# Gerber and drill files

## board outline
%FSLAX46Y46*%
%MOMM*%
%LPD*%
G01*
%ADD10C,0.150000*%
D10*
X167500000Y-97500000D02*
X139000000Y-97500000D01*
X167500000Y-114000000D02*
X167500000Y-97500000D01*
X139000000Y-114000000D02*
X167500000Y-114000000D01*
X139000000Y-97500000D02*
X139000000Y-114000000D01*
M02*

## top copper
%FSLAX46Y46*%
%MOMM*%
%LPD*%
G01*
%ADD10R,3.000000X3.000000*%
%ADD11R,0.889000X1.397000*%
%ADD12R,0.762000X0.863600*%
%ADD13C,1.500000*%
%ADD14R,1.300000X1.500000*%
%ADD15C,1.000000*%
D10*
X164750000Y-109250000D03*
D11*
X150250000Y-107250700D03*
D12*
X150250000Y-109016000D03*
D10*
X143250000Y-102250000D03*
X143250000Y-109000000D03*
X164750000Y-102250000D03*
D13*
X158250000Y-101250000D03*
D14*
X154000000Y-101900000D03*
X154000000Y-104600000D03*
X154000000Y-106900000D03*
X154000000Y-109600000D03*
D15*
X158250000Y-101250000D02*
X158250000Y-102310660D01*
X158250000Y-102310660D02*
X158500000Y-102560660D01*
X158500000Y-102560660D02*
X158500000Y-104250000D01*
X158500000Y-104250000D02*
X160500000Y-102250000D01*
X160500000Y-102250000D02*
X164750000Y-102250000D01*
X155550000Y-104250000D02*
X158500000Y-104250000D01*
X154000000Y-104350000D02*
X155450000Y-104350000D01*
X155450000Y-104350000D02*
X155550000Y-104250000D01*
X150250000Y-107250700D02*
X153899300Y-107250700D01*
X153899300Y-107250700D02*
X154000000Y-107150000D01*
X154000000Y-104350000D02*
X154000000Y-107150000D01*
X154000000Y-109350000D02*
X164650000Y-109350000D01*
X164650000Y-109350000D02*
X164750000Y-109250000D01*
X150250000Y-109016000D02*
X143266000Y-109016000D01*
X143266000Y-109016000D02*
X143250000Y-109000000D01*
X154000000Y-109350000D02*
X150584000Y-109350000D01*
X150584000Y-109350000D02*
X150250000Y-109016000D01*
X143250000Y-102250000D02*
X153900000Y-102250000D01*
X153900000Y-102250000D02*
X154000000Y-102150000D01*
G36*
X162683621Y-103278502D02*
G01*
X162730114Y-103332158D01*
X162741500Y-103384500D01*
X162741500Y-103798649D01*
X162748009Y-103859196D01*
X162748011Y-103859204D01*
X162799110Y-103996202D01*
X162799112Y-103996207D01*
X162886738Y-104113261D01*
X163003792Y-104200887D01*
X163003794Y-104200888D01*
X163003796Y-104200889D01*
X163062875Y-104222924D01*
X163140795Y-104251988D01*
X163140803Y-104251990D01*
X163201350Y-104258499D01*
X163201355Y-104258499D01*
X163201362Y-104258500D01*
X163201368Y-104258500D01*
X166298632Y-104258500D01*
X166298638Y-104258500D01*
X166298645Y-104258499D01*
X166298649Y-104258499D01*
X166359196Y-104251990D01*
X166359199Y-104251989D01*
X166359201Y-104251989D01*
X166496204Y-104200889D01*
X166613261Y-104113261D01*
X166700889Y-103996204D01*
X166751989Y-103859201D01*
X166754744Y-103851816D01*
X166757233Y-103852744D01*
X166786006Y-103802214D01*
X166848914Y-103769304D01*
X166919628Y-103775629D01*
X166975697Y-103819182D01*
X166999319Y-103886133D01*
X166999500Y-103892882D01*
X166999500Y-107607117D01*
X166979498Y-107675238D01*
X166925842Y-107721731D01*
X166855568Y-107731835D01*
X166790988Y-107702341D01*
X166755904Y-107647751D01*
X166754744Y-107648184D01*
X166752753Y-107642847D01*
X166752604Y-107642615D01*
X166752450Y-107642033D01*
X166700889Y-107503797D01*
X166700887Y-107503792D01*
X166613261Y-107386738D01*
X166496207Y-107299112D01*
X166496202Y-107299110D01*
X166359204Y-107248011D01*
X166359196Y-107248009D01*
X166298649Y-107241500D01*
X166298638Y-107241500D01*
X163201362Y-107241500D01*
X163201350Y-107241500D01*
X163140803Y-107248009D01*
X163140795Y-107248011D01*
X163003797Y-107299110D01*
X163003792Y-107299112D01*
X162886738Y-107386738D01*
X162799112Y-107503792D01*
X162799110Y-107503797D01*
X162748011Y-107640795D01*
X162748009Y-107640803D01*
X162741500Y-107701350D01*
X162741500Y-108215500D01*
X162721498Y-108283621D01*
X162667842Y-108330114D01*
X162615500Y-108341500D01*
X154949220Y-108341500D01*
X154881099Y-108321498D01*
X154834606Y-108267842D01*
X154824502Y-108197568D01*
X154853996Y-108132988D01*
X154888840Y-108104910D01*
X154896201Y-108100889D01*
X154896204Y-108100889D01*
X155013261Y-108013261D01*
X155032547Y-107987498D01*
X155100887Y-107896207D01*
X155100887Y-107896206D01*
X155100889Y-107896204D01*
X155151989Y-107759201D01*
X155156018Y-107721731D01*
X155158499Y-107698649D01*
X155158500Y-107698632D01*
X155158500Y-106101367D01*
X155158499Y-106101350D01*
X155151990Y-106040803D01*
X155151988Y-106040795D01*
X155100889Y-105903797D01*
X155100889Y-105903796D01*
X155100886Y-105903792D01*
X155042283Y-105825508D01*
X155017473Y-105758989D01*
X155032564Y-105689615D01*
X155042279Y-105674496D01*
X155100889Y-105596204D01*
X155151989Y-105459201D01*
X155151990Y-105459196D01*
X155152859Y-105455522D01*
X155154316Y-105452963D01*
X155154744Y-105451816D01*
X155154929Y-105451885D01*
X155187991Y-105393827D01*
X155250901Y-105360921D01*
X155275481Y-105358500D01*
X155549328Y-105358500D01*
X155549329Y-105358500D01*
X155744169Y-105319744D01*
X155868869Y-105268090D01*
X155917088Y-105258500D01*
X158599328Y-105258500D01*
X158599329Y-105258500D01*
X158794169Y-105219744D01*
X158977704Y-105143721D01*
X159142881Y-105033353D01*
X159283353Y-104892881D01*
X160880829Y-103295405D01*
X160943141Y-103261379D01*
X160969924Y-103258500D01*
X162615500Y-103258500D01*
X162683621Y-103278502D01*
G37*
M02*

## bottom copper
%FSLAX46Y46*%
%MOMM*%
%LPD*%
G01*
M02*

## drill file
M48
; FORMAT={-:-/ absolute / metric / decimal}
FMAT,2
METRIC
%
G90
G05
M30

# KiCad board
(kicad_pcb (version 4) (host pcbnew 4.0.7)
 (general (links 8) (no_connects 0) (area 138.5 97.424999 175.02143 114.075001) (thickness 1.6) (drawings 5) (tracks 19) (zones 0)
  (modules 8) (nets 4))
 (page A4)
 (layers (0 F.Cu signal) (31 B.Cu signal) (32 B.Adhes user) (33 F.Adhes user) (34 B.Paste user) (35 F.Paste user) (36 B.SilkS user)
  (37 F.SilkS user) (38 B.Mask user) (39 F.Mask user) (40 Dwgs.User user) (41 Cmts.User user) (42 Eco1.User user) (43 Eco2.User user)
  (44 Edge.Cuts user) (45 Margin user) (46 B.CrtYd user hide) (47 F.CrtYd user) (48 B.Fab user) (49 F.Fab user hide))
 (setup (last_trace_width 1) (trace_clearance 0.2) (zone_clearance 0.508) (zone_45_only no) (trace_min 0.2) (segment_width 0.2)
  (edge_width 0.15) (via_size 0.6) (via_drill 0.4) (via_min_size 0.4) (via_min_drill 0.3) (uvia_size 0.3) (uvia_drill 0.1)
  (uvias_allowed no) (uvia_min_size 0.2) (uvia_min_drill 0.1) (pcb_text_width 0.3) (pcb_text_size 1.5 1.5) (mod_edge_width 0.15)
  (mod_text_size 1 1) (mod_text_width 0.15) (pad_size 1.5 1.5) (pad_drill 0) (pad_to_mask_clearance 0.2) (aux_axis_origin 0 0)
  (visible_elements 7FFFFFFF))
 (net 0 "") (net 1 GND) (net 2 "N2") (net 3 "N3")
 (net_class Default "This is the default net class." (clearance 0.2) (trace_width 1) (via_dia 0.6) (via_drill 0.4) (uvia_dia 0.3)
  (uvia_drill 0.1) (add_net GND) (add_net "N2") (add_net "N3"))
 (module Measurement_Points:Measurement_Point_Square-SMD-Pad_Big (layer F.Cu) (at 164.75 109.25)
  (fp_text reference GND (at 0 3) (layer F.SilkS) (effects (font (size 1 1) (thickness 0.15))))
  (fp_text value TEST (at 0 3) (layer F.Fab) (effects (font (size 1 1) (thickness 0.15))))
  (pad 1 smd rect (at 0 0) (size 3 3) (layers F.Cu F.Mask) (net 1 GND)))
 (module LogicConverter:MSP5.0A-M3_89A (layer F.Cu) (at 150.25 108 270)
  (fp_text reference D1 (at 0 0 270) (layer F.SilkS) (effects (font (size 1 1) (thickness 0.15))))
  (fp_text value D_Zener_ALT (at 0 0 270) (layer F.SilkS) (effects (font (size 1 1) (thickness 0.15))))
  (pad 1 smd rect (at -0.7493 0 270) (size 1.397 0.889) (layers F.Cu F.Paste F.Mask) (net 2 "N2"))
  (pad 2 smd rect (at 1.016 0 270) (size 0.8636 0.762) (layers F.Cu F.Paste F.Mask) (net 1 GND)))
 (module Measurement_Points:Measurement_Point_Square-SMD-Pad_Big (layer F.Cu) (at 143.25 102.25)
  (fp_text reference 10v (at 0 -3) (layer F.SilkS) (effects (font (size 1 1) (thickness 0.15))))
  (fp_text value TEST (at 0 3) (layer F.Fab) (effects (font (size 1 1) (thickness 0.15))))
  (pad 1 smd rect (at 0 0) (size 3 3) (layers F.Cu F.Mask) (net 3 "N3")))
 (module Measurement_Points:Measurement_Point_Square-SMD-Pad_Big (layer F.Cu) (at 143.25 109)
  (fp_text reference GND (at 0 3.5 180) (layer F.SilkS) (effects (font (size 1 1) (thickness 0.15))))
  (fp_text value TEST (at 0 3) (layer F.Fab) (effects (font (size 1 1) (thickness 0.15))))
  (pad 1 smd rect (at 0 0) (size 3 3) (layers F.Cu F.Mask) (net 1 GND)))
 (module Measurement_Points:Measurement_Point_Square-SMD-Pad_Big (layer F.Cu) (at 164.75 102.25)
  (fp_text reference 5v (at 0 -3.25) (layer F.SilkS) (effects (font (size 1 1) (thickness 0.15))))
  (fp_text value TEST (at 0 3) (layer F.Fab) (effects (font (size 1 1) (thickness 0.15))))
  (pad 1 smd rect (at 0 0) (size 3 3) (layers F.Cu F.Mask) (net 2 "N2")))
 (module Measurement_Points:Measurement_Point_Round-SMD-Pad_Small (layer F.Cu) (at 158.25 101.25)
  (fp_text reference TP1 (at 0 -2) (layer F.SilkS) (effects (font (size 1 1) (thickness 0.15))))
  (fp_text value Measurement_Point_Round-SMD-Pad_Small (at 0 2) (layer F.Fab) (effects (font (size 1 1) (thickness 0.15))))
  (pad 1 smd circle (at 0 0) (size 1.5 1.5) (layers F.Cu F.Mask) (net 2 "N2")))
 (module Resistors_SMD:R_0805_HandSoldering (layer F.Cu) (at 154 103.25 270)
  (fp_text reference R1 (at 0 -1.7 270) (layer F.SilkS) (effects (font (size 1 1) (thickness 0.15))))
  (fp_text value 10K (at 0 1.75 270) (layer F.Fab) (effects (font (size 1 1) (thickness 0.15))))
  (pad 1 smd rect (at -1.35 0 270) (size 1.5 1.3) (layers F.Cu F.Paste F.Mask) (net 3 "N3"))
  (pad 2 smd rect (at 1.35 0 270) (size 1.5 1.3) (layers F.Cu F.Paste F.Mask) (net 2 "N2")))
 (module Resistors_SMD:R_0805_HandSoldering (layer F.Cu) (at 154 108.25 270)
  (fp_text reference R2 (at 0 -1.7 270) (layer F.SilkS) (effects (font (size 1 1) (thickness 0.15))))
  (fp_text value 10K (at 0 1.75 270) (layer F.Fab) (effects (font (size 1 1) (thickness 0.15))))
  (pad 1 smd rect (at -1.35 0 270) (size 1.5 1.3) (layers F.Cu F.Paste F.Mask) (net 2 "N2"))
  (pad 2 smd rect (at 1.35 0 270) (size 1.5 1.3) (layers F.Cu F.Paste F.Mask) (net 1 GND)))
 (gr_line (start 167.5 97.5) (end 139 97.5) (layer Edge.Cuts) (width 0.15))
 (gr_line (start 167.5 114) (end 167.5 97.5) (layer Edge.Cuts) (width 0.15))
 (gr_line (start 139 114) (end 167.5 114) (layer Edge.Cuts) (width 0.15))
 (gr_line (start 139 97.5) (end 139 114) (layer Edge.Cuts) (width 0.15))
 (segment (start 158.25 101.25) (end 158.25 102.31066) (width 1) (layer F.Cu) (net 2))
 (segment (start 158.25 102.31066) (end 158.5 102.56066) (width 1) (layer F.Cu) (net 2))
 (segment (start 158.5 102.56066) (end 158.5 104.25) (width 1) (layer F.Cu) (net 2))
 (segment (start 158.5 104.25) (end 160.5 102.25) (width 1) (layer F.Cu) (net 2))
 (segment (start 160.5 102.25) (end 164.75 102.25) (width 1) (layer F.Cu) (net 2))
 (segment (start 155.55 104.25) (end 158.5 104.25) (width 1) (layer F.Cu) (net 2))
 (segment (start 154 104.35) (end 155.45 104.35) (width 1) (layer F.Cu) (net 2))
 (segment (start 155.45 104.35) (end 155.55 104.25) (width 1) (layer F.Cu) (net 2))
 (segment (start 150.25 107.2507) (end 153.8993 107.2507) (width 1) (layer F.Cu) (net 2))
 (segment (start 153.8993 107.2507) (end 154 107.15) (width 1) (layer F.Cu) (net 2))
 (segment (start 154 104.35) (end 154 107.15) (width 1) (layer F.Cu) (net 2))
 (segment (start 154 109.35) (end 164.65 109.35) (width 1) (layer F.Cu) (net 1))
 (segment (start 164.65 109.35) (end 164.75 109.25) (width 1) (layer F.Cu) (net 1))
 (segment (start 150.25 109.016) (end 143.266 109.016) (width 1) (layer F.Cu) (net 1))
 (segment (start 143.266 109.016) (end 143.25 109) (width 1) (layer F.Cu) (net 1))
 (segment (start 154 109.35) (end 150.584 109.35) (width 1) (layer F.Cu) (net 1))
 (segment (start 150.584 109.35) (end 150.25 109.016) (width 1) (layer F.Cu) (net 1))
 (segment (start 143.25 102.25) (end 153.9 102.25) (width 1) (layer F.Cu) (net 3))
 (segment (start 153.9 102.25) (end 154 102.15) (width 1) (layer F.Cu) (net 3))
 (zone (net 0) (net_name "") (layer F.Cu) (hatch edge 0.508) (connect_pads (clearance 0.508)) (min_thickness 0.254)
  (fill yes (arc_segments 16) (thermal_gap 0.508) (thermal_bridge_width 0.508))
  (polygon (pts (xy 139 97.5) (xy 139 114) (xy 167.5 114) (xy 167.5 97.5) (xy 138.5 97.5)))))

